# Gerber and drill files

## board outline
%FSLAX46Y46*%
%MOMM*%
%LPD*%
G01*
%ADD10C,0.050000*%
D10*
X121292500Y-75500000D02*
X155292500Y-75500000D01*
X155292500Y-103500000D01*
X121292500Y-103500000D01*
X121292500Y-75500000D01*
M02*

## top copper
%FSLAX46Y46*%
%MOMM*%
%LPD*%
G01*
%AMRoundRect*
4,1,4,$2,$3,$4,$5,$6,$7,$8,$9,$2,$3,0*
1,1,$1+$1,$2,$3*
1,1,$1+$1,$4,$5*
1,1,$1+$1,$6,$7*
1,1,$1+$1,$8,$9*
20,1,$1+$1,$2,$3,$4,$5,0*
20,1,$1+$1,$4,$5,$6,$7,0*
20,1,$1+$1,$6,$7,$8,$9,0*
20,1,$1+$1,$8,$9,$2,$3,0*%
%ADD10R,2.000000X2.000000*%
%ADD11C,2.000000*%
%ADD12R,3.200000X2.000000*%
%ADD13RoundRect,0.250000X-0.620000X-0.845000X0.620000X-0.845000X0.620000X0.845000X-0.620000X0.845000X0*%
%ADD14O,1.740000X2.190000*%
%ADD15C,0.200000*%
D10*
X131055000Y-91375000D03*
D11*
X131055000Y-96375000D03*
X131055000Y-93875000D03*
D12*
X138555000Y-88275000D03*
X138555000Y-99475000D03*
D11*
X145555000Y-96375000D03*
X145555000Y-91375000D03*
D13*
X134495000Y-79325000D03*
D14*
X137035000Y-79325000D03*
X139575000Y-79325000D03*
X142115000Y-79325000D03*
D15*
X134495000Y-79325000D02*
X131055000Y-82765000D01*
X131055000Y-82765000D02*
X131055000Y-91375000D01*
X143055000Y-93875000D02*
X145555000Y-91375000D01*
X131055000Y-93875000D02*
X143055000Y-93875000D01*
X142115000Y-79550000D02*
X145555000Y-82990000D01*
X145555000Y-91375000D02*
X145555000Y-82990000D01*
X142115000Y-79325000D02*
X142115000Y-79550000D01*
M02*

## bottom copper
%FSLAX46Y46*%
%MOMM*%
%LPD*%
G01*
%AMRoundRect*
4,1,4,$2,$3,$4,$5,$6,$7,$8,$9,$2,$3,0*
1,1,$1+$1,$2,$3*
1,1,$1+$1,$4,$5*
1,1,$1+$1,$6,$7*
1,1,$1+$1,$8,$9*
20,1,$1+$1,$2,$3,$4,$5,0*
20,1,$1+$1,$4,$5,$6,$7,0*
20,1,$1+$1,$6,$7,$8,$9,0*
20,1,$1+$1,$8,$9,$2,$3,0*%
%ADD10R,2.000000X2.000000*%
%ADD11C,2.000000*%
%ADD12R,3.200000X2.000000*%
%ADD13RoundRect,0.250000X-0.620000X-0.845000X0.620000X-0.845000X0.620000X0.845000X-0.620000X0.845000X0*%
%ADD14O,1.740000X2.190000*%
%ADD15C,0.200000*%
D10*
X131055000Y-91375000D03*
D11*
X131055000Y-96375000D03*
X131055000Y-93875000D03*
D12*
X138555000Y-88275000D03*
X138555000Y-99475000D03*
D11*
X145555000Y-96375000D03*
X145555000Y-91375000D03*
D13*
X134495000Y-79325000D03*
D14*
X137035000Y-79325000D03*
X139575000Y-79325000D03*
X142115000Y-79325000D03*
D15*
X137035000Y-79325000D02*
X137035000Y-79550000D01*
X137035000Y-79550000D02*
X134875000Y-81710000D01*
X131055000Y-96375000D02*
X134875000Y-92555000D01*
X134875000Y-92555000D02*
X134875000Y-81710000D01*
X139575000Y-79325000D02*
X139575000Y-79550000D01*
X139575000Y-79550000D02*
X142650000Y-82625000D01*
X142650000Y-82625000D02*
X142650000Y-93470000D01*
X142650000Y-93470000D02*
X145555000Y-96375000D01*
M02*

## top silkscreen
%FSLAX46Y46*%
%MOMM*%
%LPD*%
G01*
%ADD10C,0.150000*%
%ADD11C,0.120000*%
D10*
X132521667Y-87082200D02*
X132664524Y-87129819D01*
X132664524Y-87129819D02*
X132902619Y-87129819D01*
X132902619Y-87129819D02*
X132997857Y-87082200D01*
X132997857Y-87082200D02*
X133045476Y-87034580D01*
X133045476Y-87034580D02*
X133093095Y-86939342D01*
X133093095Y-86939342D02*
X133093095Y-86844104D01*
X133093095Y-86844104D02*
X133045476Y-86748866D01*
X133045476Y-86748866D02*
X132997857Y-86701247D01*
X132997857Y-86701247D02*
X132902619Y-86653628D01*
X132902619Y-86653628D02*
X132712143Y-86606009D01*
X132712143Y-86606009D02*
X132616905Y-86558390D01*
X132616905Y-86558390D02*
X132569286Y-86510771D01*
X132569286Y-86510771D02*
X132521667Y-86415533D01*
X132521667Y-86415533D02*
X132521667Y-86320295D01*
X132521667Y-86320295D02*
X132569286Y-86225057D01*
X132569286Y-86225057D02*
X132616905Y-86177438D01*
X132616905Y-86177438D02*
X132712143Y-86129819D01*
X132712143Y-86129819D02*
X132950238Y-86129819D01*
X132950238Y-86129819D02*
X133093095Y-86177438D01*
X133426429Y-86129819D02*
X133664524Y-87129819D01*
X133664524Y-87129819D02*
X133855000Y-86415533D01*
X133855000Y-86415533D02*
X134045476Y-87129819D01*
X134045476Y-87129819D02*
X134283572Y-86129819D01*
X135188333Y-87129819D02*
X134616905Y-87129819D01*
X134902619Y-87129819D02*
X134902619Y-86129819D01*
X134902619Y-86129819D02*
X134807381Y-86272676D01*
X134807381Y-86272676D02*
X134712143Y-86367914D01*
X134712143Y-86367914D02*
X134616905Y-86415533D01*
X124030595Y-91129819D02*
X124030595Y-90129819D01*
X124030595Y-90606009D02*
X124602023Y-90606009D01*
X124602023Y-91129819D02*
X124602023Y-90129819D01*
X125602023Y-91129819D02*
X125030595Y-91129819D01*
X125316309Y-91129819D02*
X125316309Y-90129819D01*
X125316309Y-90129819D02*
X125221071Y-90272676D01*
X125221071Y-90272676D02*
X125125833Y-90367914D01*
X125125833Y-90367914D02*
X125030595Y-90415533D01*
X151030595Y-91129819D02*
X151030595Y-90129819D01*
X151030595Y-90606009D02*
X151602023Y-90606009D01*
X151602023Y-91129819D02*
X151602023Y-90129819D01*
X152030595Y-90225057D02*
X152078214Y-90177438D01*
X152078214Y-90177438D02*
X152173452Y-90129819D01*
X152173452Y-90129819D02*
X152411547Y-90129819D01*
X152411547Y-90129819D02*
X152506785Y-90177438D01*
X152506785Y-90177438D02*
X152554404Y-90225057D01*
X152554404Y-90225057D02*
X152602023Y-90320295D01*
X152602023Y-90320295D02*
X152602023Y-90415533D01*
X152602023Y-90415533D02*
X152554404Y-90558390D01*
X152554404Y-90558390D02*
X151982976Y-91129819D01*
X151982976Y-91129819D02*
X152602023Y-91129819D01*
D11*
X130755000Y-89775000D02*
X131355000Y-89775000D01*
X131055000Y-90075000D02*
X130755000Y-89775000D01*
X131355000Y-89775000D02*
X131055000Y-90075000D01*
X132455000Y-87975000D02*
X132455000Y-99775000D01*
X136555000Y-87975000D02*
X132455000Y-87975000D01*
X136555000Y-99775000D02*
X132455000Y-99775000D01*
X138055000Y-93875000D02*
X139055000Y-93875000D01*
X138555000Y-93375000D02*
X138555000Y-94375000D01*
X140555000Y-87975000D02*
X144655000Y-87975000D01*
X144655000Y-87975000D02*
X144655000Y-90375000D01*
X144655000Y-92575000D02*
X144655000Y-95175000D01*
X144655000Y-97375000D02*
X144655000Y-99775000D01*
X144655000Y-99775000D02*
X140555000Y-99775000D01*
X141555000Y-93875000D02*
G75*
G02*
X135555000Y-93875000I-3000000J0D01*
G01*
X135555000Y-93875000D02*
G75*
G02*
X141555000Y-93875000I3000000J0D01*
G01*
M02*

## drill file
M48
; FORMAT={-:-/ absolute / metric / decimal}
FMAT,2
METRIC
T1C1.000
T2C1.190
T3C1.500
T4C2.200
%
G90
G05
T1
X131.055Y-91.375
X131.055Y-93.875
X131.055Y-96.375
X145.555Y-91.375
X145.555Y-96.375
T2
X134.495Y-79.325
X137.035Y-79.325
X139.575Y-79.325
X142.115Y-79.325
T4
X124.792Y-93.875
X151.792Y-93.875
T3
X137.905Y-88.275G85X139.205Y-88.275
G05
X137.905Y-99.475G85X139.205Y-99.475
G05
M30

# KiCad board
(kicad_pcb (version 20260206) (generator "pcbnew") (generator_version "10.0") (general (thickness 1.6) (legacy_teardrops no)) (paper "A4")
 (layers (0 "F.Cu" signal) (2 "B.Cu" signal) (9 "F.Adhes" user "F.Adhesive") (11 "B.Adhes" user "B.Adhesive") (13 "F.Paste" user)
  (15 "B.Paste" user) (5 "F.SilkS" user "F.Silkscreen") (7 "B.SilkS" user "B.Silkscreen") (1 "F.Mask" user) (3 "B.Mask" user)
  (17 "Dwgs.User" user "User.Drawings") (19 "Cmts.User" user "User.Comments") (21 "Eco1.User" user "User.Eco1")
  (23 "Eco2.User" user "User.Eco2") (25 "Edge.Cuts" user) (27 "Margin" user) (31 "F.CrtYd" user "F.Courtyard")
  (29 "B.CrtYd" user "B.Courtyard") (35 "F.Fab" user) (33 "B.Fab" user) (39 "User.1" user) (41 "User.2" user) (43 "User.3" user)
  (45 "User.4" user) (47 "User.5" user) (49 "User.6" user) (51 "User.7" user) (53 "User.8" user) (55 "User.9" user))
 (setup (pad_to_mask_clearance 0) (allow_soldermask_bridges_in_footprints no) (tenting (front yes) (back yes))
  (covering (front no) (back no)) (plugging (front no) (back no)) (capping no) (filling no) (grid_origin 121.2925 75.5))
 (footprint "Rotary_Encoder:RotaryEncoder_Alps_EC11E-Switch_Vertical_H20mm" (layer "F.Cu") (at 131.055 91.375)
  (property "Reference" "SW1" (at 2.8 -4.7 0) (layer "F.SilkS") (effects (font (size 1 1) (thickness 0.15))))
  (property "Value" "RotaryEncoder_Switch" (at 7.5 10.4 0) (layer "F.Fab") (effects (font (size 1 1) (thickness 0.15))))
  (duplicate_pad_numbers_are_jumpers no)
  (fp_line (start -0.3 -1.6) (end 0.3 -1.6) (stroke (width 0.12) (type solid)) (layer "F.SilkS"))
  (fp_line (start 0 -1.3) (end -0.3 -1.6) (stroke (width 0.12) (type solid)) (layer "F.SilkS"))
  (fp_line (start 0.3 -1.6) (end 0 -1.3) (stroke (width 0.12) (type solid)) (layer "F.SilkS"))
  (fp_line (start 1.4 -3.4) (end 1.4 8.4) (stroke (width 0.12) (type solid)) (layer "F.SilkS"))
  (fp_line (start 5.5 -3.4) (end 1.4 -3.4) (stroke (width 0.12) (type solid)) (layer "F.SilkS"))
  (fp_line (start 5.5 8.4) (end 1.4 8.4) (stroke (width 0.12) (type solid)) (layer "F.SilkS"))
  (fp_line (start 7 2.5) (end 8 2.5) (stroke (width 0.12) (type solid)) (layer "F.SilkS"))
  (fp_line (start 7.5 2) (end 7.5 3) (stroke (width 0.12) (type solid)) (layer "F.SilkS"))
  (fp_line (start 9.5 -3.4) (end 13.6 -3.4) (stroke (width 0.12) (type solid)) (layer "F.SilkS"))
  (fp_line (start 13.6 -3.4) (end 13.6 -1) (stroke (width 0.12) (type solid)) (layer "F.SilkS"))
  (fp_line (start 13.6 1.2) (end 13.6 3.8) (stroke (width 0.12) (type solid)) (layer "F.SilkS"))
  (fp_line (start 13.6 6) (end 13.6 8.4) (stroke (width 0.12) (type solid)) (layer "F.SilkS"))
  (fp_line (start 13.6 8.4) (end 9.5 8.4) (stroke (width 0.12) (type solid)) (layer "F.SilkS"))
  (fp_circle (center 7.5 2.5) (end 10.5 2.5) (stroke (width 0.12) (type solid)) (fill no) (layer "F.SilkS"))
  (pad "A" thru_hole rect (at 0 0) (size 2 2) (drill 1) (layers "*.Cu" "*.Mask") (remove_unused_layers no) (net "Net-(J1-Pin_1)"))
  (pad "B" thru_hole circle (at 0 5) (size 2 2) (drill 1) (layers "*.Cu" "*.Mask") (remove_unused_layers no) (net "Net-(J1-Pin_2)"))
  (pad "C" thru_hole circle (at 0 2.5) (size 2 2) (drill 1) (layers "*.Cu" "*.Mask") (remove_unused_layers no) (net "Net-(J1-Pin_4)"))
  (pad "MP" thru_hole rect (at 7.5 -3.1) (size 3.2 2) (drill oval 2.8 1.5) (layers "*.Cu" "*.Mask") (remove_unused_layers no))
  (pad "MP" thru_hole rect (at 7.5 8.1) (size 3.2 2) (drill oval 2.8 1.5) (layers "*.Cu" "*.Mask") (remove_unused_layers no))
  (pad "S1" thru_hole circle (at 14.5 5) (size 2 2) (drill 1) (layers "*.Cu" "*.Mask") (remove_unused_layers no) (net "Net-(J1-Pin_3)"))
  (pad "S2" thru_hole circle (at 14.5 0) (size 2 2) (drill 1) (layers "*.Cu" "*.Mask") (remove_unused_layers no) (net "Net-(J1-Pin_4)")))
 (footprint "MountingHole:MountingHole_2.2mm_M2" (layer "F.Cu") (at 124.7925 93.875)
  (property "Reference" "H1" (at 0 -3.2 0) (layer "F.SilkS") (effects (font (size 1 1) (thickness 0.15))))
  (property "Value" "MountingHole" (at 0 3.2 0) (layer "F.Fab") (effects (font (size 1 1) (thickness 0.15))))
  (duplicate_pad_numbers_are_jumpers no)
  (pad "" np_thru_hole circle (at 0 0) (size 2.2 2.2) (drill 2.2) (layers "*.Cu" "*.Mask")))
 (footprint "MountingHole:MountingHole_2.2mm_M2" (layer "F.Cu") (at 151.7925 93.875)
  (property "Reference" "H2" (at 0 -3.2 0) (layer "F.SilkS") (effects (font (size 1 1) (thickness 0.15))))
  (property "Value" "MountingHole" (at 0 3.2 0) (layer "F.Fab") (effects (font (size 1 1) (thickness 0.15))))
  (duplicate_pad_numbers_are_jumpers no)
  (pad "" np_thru_hole circle (at 0 0) (size 2.2 2.2) (drill 2.2) (layers "*.Cu" "*.Mask")))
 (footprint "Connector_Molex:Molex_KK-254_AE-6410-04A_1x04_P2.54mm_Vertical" (layer "B.Cu") (at 134.495 79.325)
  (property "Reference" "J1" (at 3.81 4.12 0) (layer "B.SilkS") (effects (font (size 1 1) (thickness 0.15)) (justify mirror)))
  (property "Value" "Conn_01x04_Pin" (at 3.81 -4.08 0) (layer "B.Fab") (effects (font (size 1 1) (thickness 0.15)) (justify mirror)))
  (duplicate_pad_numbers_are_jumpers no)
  (pad "1" thru_hole roundrect (at 0 0) (size 1.74 2.19) (drill 1.19) (layers "*.Cu" "*.Mask") (remove_unused_layers no)
   (roundrect_rratio 0.1436781609) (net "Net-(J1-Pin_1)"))
  (pad "2" thru_hole oval (at 2.54 0) (size 1.74 2.19) (drill 1.19) (layers "*.Cu" "*.Mask") (remove_unused_layers no)
   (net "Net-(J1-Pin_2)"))
  (pad "3" thru_hole oval (at 5.08 0) (size 1.74 2.19) (drill 1.19) (layers "*.Cu" "*.Mask") (remove_unused_layers no)
   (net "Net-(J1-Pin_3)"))
  (pad "4" thru_hole oval (at 7.62 0) (size 1.74 2.19) (drill 1.19) (layers "*.Cu" "*.Mask") (remove_unused_layers no)
   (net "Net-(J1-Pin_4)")))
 (gr_rect (start 121.2925 75.5) (end 155.2925 103.5) (stroke (width 0.05) (type default)) (fill no) (layer "Edge.Cuts"))
 (segment (start 134.495 79.325) (end 131.055 82.765) (width 0.2) (layer "F.Cu") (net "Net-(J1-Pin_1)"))
 (segment (start 131.055 82.765) (end 131.055 91.375) (width 0.2) (layer "F.Cu") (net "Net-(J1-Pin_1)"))
 (segment (start 137.035 79.325) (end 137.035 79.55) (width 0.2) (layer "B.Cu") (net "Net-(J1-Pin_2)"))
 (segment (start 137.035 79.55) (end 134.875 81.71) (width 0.2) (layer "B.Cu") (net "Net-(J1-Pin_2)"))
 (segment (start 131.055 96.375) (end 134.875 92.555) (width 0.2) (layer "B.Cu") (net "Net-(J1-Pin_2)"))
 (segment (start 134.875 92.555) (end 134.875 81.71) (width 0.2) (layer "B.Cu") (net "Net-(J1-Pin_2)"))
 (segment (start 139.575 79.325) (end 139.575 79.55) (width 0.2) (layer "B.Cu") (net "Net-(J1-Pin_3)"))
 (segment (start 139.575 79.55) (end 142.65 82.625) (width 0.2) (layer "B.Cu") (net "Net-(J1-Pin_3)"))
 (segment (start 142.65 82.625) (end 142.65 93.47) (width 0.2) (layer "B.Cu") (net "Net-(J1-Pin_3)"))
 (segment (start 142.65 93.47) (end 145.555 96.375) (width 0.2) (layer "B.Cu") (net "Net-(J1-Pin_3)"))
 (segment (start 143.055 93.875) (end 145.555 91.375) (width 0.2) (layer "F.Cu") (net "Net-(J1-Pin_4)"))
 (segment (start 131.055 93.875) (end 143.055 93.875) (width 0.2) (layer "F.Cu") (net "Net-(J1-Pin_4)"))
 (segment (start 142.115 79.55) (end 145.555 82.99) (width 0.2) (layer "F.Cu") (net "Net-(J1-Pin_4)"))
 (segment (start 145.555 91.375) (end 145.555 82.99) (width 0.2) (layer "F.Cu") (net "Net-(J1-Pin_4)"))
 (segment (start 142.115 79.325) (end 142.115 79.55) (width 0.2) (layer "F.Cu") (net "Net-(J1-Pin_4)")))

